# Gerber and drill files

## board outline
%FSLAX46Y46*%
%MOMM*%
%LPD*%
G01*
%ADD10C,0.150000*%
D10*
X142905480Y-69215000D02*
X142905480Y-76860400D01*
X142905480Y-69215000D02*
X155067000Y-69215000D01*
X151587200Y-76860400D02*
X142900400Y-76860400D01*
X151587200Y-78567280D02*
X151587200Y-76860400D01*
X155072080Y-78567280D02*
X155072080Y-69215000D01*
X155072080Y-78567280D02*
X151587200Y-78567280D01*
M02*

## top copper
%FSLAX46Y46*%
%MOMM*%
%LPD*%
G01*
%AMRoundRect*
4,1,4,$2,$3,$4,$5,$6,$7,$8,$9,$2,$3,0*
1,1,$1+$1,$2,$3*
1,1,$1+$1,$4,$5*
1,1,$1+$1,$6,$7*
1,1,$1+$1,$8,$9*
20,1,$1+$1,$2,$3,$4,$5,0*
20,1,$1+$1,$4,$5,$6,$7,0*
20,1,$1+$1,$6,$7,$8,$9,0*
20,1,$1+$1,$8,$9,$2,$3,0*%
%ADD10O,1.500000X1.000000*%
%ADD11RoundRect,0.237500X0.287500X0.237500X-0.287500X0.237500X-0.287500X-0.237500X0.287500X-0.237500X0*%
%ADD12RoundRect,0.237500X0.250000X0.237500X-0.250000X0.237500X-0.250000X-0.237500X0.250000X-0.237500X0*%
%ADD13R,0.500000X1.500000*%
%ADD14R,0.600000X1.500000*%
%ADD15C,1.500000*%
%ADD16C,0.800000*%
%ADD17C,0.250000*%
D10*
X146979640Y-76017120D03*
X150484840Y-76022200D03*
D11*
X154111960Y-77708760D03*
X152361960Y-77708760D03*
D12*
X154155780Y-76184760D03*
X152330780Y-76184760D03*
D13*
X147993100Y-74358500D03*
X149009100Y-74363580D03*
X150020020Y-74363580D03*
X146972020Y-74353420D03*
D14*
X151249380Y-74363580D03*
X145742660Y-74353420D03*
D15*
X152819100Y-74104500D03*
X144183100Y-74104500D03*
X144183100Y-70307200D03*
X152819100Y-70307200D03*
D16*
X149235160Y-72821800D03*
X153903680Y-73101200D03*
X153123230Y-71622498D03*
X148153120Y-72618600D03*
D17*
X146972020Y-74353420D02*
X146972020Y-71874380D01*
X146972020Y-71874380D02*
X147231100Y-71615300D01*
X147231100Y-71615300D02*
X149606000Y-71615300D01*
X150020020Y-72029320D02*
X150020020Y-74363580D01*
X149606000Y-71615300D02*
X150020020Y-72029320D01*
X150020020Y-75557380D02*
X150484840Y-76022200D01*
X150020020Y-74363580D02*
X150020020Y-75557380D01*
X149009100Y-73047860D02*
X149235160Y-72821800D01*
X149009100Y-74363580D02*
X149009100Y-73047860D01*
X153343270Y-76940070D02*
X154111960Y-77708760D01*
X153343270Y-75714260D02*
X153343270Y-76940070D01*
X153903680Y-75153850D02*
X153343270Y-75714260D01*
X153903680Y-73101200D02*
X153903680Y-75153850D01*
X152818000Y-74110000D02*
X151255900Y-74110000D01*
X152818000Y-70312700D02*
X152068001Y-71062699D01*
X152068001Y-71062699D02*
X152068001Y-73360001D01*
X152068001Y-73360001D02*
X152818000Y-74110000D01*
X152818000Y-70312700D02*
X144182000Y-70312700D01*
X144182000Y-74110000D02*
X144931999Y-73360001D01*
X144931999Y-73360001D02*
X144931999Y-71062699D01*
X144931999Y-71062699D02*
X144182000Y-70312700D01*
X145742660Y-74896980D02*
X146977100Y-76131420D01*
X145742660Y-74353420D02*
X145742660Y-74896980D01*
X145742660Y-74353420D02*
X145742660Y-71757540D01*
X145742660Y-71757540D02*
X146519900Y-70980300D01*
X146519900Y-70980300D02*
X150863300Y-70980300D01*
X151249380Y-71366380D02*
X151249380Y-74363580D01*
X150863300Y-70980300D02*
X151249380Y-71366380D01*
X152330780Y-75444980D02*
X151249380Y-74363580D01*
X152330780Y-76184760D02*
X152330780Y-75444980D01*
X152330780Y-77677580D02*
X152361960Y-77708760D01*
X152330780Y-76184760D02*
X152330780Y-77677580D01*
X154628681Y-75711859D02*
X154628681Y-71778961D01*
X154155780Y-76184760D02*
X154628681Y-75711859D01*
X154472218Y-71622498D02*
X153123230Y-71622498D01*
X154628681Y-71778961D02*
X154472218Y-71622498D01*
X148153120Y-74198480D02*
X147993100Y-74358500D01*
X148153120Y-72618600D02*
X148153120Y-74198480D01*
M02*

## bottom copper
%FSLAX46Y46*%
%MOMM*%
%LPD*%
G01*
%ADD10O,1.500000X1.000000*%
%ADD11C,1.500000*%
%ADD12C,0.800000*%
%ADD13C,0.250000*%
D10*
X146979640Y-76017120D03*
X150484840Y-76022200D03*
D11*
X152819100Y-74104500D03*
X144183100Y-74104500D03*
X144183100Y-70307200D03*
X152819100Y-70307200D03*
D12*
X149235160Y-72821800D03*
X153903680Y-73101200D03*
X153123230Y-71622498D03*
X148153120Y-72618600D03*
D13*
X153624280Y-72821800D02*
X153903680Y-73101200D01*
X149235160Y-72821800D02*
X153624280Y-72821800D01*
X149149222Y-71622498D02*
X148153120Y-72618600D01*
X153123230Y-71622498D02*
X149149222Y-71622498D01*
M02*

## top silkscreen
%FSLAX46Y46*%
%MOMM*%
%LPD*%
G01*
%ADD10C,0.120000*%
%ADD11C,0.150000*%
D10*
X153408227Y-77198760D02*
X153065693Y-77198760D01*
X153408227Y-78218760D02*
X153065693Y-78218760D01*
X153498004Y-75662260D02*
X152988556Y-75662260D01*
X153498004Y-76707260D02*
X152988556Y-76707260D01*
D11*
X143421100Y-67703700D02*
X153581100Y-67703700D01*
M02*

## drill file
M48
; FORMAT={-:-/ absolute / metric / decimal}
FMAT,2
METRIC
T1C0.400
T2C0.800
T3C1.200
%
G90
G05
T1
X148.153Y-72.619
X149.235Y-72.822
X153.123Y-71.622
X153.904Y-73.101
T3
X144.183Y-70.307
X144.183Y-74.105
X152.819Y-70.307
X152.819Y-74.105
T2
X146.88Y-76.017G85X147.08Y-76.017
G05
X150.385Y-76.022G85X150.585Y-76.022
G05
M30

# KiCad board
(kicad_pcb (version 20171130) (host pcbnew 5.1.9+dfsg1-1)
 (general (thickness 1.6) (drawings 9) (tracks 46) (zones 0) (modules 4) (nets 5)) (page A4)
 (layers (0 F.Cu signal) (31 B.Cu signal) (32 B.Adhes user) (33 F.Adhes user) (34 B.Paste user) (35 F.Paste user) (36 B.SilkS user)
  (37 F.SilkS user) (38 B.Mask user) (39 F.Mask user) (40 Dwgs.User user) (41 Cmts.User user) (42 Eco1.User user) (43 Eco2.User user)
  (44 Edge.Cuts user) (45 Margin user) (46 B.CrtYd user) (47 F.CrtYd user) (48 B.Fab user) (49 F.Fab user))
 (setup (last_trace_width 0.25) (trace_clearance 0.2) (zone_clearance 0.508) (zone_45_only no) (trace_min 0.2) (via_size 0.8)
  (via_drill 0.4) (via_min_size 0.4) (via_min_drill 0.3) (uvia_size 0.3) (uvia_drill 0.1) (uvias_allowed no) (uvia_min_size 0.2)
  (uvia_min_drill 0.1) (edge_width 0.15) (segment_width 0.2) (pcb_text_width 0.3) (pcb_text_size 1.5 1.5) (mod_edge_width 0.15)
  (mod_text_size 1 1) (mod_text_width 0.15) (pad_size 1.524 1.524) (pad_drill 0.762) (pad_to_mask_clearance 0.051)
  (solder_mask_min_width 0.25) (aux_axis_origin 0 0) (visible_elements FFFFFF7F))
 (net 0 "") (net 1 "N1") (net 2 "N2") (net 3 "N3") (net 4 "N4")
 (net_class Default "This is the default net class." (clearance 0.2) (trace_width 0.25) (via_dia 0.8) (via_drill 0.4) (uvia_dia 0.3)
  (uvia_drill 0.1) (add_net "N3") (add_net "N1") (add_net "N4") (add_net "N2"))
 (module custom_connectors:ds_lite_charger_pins (layer F.Cu) (at 148.73224 76.0222)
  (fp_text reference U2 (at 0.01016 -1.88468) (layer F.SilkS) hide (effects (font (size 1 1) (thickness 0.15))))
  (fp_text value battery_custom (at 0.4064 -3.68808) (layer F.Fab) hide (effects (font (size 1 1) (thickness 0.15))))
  (pad 1 thru_hole oval (at -1.7526 -0.00508 90) (size 1 1.5) (drill oval 0.8 1) (layers *.Cu *.Mask) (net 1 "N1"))
  (pad 2 thru_hole oval (at 1.7526 0 90) (size 1 1.5) (drill oval 0.8 1) (layers *.Cu *.Mask) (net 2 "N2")))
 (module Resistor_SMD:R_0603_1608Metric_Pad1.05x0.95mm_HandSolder (layer F.Cu) (at 153.23696 77.70876 180)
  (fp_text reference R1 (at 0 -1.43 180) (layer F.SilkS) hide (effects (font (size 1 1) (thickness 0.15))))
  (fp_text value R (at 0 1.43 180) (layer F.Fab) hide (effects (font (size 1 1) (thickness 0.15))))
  (fp_line (start -0.171267 0.51) (end 0.171267 0.51) (layer F.SilkS) (width 0.12))
  (fp_line (start -0.171267 -0.51) (end 0.171267 -0.51) (layer F.SilkS) (width 0.12))
  (pad 1 smd roundrect (at -0.875 0 180) (size 1.05 0.95) (layers F.Cu F.Paste F.Mask) (roundrect_rratio 0.25) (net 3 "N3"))
  (pad 2 smd roundrect (at 0.875 0 180) (size 1.05 0.95) (layers F.Cu F.Paste F.Mask) (roundrect_rratio 0.25) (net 1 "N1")))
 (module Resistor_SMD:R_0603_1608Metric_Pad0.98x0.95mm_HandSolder (layer F.Cu) (at 153.24328 76.18476 180)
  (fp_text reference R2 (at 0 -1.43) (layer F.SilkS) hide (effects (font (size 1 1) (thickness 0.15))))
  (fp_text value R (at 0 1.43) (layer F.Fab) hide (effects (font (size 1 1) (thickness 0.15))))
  (fp_line (start -0.254724 0.5225) (end 0.254724 0.5225) (layer F.SilkS) (width 0.12))
  (fp_line (start -0.254724 -0.5225) (end 0.254724 -0.5225) (layer F.SilkS) (width 0.12))
  (pad 1 smd roundrect (at -0.9125 0 180) (size 0.975 0.95) (layers F.Cu F.Paste F.Mask) (roundrect_rratio 0.25) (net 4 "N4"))
  (pad 2 smd roundrect (at 0.9125 0 180) (size 0.975 0.95) (layers F.Cu F.Paste F.Mask) (roundrect_rratio 0.25) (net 1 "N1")))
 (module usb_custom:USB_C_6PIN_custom (layer F.Cu) (at 148.5011 74.1045)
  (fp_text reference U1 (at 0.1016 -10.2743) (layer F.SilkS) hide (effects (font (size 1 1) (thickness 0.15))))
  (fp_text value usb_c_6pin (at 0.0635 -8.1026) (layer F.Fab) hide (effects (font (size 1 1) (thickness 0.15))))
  (fp_line (start -5.08 -6.4008) (end 5.08 -6.4008) (layer F.SilkS) (width 0.15))
  (pad 3 smd rect (at -0.508 0.254) (size 0.5 1.5) (layers F.Cu F.Paste F.Mask) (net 4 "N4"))
  (pad 4 smd rect (at 0.508 0.25908) (size 0.5 1.5) (layers F.Cu F.Paste F.Mask) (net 3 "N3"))
  (pad 2 smd rect (at 1.51892 0.25908) (size 0.5 1.5) (layers F.Cu F.Paste F.Mask) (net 2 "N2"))
  (pad 2 smd rect (at -1.52908 0.24892) (size 0.5 1.5) (layers F.Cu F.Paste F.Mask) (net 2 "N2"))
  (pad 1 smd rect (at 2.74828 0.25908) (size 0.6 1.5) (layers F.Cu F.Paste F.Mask) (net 1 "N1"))
  (pad 1 smd rect (at -2.75844 0.24892) (size 0.6 1.5) (layers F.Cu F.Paste F.Mask) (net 1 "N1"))
  (pad 1 thru_hole circle (at 4.318 0) (size 1.5 1.5) (drill 1.2) (layers *.Cu *.Mask) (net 1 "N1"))
  (pad 1 thru_hole circle (at -4.318 0) (size 1.5 1.5) (drill 1.2) (layers *.Cu *.Mask) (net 1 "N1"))
  (pad 1 thru_hole circle (at -4.318 -3.7973) (size 1.5 1.5) (drill 1.2) (layers *.Cu *.Mask) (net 1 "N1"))
  (pad 1 thru_hole circle (at 4.318 -3.7973) (size 1.5 1.5) (drill 1.2) (layers *.Cu *.Mask) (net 1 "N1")))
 (gr_line (start 142.90548 69.215) (end 142.90548 76.8604) (layer Edge.Cuts) (width 0.15))
 (gr_line (start 142.90548 69.215) (end 155.067 69.215) (layer Edge.Cuts) (width 0.15))
 (gr_line (start 151.5872 76.8604) (end 142.9004 76.8604) (layer Edge.Cuts) (width 0.15))
 (gr_line (start 151.5872 78.56728) (end 151.5872 76.8604) (layer Edge.Cuts) (width 0.15))
 (gr_line (start 155.07208 78.56728) (end 155.07208 69.215) (layer Edge.Cuts) (width 0.15))
 (gr_line (start 155.07208 78.56728) (end 151.5872 78.56728) (layer Edge.Cuts) (width 0.15))
 (segment (start 146.97202 74.35342) (end 146.97202 71.87438) (width 0.25) (layer F.Cu) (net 2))
 (segment (start 146.97202 71.87438) (end 147.2311 71.6153) (width 0.25) (layer F.Cu) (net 2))
 (segment (start 147.2311 71.6153) (end 149.606 71.6153) (width 0.25) (layer F.Cu) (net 2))
 (segment (start 150.02002 72.02932) (end 150.02002 74.36358) (width 0.25) (layer F.Cu) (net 2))
 (segment (start 149.606 71.6153) (end 150.02002 72.02932) (width 0.25) (layer F.Cu) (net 2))
 (segment (start 150.02002 75.55738) (end 150.48484 76.0222) (width 0.25) (layer F.Cu) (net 2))
 (segment (start 150.02002 74.36358) (end 150.02002 75.55738) (width 0.25) (layer F.Cu) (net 2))
 (via (at 149.23516 72.8218) (size 0.8) (drill 0.4) (layers F.Cu B.Cu) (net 3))
 (segment (start 149.0091 73.04786) (end 149.23516 72.8218) (width 0.25) (layer F.Cu) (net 3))
 (segment (start 149.0091 74.36358) (end 149.0091 73.04786) (width 0.25) (layer F.Cu) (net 3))
 (via (at 153.90368 73.1012) (size 0.8) (drill 0.4) (layers F.Cu B.Cu) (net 3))
 (segment (start 153.62428 72.8218) (end 153.90368 73.1012) (width 0.25) (layer B.Cu) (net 3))
 (segment (start 149.23516 72.8218) (end 153.62428 72.8218) (width 0.25) (layer B.Cu) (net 3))
 (segment (start 153.34327 76.94007) (end 154.11196 77.70876) (width 0.25) (layer F.Cu) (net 3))
 (segment (start 153.34327 75.71426) (end 153.34327 76.94007) (width 0.25) (layer F.Cu) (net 3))
 (segment (start 153.90368 75.15385) (end 153.34327 75.71426) (width 0.25) (layer F.Cu) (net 3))
 (segment (start 153.90368 73.1012) (end 153.90368 75.15385) (width 0.25) (layer F.Cu) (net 3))
 (segment (start 152.818 74.11) (end 151.2559 74.11) (width 0.25) (layer F.Cu) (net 1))
 (segment (start 152.818 70.3127) (end 152.068001 71.062699) (width 0.25) (layer F.Cu) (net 1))
 (segment (start 152.068001 71.062699) (end 152.068001 73.360001) (width 0.25) (layer F.Cu) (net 1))
 (segment (start 152.068001 73.360001) (end 152.818 74.11) (width 0.25) (layer F.Cu) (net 1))
 (segment (start 152.818 70.3127) (end 144.182 70.3127) (width 0.25) (layer F.Cu) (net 1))
 (segment (start 144.182 74.11) (end 144.931999 73.360001) (width 0.25) (layer F.Cu) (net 1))
 (segment (start 144.931999 73.360001) (end 144.931999 71.062699) (width 0.25) (layer F.Cu) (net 1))
 (segment (start 144.931999 71.062699) (end 144.182 70.3127) (width 0.25) (layer F.Cu) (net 1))
 (segment (start 145.74266 74.89698) (end 146.9771 76.13142) (width 0.25) (layer F.Cu) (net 1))
 (segment (start 145.74266 74.35342) (end 145.74266 74.89698) (width 0.25) (layer F.Cu) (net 1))
 (segment (start 145.74266 74.35342) (end 145.74266 71.75754) (width 0.25) (layer F.Cu) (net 1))
 (segment (start 145.74266 71.75754) (end 146.5199 70.9803) (width 0.25) (layer F.Cu) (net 1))
 (segment (start 146.5199 70.9803) (end 150.8633 70.9803) (width 0.25) (layer F.Cu) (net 1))
 (segment (start 151.24938 71.36638) (end 151.24938 74.36358) (width 0.25) (layer F.Cu) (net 1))
 (segment (start 150.8633 70.9803) (end 151.24938 71.36638) (width 0.25) (layer F.Cu) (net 1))
 (segment (start 152.33078 75.44498) (end 151.24938 74.36358) (width 0.25) (layer F.Cu) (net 1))
 (segment (start 152.33078 76.18476) (end 152.33078 75.44498) (width 0.25) (layer F.Cu) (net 1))
 (segment (start 152.33078 77.67758) (end 152.36196 77.70876) (width 0.25) (layer F.Cu) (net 1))
 (segment (start 152.33078 76.18476) (end 152.33078 77.67758) (width 0.25) (layer F.Cu) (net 1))
 (segment (start 154.628681 75.711859) (end 154.628681 71.778961) (width 0.25) (layer F.Cu) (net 4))
 (segment (start 154.15578 76.18476) (end 154.628681 75.711859) (width 0.25) (layer F.Cu) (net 4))
 (via (at 153.12323 71.622498) (size 0.8) (drill 0.4) (layers F.Cu B.Cu) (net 4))
 (segment (start 154.472218 71.622498) (end 153.12323 71.622498) (width 0.25) (layer F.Cu) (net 4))
 (segment (start 154.628681 71.778961) (end 154.472218 71.622498) (width 0.25) (layer F.Cu) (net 4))
 (via (at 148.15312 72.6186) (size 0.8) (drill 0.4) (layers F.Cu B.Cu) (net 4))
 (segment (start 149.149222 71.622498) (end 148.15312 72.6186) (width 0.25) (layer B.Cu) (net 4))
 (segment (start 153.12323 71.622498) (end 149.149222 71.622498) (width 0.25) (layer B.Cu) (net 4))
 (segment (start 148.15312 74.19848) (end 147.9931 74.3585) (width 0.25) (layer F.Cu) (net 4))
 (segment (start 148.15312 72.6186) (end 148.15312 74.19848) (width 0.25) (layer F.Cu) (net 4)))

